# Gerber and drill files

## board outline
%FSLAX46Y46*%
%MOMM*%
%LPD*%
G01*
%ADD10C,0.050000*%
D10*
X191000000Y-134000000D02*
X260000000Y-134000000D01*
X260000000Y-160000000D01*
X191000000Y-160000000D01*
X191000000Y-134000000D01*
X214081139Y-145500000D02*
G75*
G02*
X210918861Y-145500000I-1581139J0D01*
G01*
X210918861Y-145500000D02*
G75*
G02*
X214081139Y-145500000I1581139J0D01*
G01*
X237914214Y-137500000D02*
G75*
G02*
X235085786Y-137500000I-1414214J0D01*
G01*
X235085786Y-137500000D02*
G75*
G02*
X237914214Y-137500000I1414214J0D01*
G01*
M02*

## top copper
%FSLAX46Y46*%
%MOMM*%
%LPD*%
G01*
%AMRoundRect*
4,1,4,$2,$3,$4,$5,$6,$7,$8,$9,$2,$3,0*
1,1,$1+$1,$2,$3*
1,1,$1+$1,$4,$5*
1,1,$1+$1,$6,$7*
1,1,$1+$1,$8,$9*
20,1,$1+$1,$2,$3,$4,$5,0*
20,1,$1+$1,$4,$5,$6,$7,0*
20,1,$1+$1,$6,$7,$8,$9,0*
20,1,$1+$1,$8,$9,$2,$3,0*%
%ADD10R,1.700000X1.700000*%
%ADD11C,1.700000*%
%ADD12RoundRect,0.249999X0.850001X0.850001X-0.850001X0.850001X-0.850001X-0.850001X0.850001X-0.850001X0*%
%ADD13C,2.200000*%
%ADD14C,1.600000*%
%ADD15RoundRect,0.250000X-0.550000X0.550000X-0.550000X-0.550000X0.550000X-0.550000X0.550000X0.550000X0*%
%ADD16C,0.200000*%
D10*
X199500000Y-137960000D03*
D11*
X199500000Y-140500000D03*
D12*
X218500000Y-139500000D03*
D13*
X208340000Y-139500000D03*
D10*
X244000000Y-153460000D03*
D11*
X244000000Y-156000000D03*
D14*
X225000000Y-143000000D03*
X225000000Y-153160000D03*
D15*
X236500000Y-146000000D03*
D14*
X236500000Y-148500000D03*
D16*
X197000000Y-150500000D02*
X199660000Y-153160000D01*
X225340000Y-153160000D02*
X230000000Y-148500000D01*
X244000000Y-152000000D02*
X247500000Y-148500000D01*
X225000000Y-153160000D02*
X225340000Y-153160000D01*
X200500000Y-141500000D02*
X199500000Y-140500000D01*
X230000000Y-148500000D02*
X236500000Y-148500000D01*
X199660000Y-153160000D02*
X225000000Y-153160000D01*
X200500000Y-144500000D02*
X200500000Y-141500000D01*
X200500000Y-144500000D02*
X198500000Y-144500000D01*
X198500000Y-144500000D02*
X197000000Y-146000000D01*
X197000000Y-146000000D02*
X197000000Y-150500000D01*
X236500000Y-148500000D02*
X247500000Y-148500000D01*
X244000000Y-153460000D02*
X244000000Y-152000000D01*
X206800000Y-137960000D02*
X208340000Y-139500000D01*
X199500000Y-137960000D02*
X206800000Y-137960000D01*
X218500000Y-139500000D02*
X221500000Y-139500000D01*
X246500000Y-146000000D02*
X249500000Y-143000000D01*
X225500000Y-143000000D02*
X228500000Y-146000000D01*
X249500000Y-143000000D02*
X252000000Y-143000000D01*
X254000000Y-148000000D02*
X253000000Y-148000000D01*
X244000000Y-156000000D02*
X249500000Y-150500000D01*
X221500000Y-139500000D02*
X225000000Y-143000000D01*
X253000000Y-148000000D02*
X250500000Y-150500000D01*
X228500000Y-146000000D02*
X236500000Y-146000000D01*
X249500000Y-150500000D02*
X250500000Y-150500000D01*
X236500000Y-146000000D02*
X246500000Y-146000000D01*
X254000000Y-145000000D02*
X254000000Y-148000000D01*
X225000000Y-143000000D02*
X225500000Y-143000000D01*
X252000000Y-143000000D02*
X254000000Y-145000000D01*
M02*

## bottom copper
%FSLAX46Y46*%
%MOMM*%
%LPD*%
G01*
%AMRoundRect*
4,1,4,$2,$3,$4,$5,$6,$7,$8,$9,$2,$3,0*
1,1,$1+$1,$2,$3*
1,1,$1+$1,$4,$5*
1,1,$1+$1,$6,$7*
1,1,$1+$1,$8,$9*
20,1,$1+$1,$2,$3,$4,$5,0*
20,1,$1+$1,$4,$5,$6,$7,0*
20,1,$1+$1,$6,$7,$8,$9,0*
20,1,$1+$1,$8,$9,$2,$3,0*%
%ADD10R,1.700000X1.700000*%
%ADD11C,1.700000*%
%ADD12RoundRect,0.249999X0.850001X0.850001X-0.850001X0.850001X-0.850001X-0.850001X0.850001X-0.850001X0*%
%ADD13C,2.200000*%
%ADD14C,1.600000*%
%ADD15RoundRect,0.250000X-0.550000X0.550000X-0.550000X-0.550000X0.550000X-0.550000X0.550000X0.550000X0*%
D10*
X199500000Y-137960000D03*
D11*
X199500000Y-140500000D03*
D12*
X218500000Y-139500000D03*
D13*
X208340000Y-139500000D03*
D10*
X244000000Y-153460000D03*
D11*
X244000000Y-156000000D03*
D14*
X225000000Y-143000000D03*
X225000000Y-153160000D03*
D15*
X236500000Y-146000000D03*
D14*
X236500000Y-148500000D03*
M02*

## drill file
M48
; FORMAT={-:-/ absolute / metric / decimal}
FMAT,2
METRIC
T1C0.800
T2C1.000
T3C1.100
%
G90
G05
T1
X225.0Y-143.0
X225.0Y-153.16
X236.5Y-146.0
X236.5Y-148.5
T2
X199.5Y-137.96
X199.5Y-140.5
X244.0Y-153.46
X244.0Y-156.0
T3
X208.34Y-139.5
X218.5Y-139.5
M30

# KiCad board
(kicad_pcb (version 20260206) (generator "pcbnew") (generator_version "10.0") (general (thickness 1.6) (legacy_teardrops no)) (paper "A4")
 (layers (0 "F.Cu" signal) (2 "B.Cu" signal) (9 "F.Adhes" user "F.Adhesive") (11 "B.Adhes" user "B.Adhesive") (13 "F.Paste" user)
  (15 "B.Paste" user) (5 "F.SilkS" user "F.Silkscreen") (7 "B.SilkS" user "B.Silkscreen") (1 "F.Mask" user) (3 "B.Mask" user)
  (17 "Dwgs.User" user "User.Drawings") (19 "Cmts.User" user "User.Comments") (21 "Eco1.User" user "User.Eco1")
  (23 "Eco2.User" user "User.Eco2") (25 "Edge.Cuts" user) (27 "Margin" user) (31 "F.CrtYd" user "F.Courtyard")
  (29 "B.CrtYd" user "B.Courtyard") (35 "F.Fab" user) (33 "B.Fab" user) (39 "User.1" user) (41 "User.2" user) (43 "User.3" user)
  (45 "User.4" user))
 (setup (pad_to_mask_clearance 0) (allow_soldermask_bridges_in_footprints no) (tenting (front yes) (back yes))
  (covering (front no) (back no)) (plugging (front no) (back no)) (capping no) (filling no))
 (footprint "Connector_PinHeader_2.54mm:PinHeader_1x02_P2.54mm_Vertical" (layer "F.Cu") (at 199.5 137.96)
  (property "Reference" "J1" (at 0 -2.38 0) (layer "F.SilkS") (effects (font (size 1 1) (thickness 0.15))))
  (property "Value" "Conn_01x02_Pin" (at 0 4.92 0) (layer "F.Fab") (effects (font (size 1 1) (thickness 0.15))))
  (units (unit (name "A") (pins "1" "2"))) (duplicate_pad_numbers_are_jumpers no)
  (pad "1" thru_hole rect (at 0 0) (size 1.7 1.7) (drill 1) (layers "*.Cu" "*.Mask") (remove_unused_layers no) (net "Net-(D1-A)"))
  (pad "2" thru_hole circle (at 0 2.54) (size 1.7 1.7) (drill 1) (layers "*.Cu" "*.Mask") (remove_unused_layers no) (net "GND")))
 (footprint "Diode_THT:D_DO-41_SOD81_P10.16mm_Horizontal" (layer "F.Cu") (at 218.5 139.5 180)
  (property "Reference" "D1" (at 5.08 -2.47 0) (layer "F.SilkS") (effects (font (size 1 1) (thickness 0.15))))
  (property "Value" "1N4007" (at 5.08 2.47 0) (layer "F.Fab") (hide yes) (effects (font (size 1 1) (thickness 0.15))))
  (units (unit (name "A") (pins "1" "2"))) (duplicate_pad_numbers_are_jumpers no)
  (pad "1" thru_hole roundrect (at 0 0 180) (size 2.2 2.2) (drill 1.1) (layers "*.Cu" "*.Mask") (remove_unused_layers no)
   (roundrect_rratio 0.113636) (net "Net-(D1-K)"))
  (pad "2" thru_hole circle (at 10.16 0 180) (size 2.2 2.2) (drill 1.1) (layers "*.Cu" "*.Mask") (remove_unused_layers no)
   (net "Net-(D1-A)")))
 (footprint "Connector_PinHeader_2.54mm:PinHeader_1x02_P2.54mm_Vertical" (layer "F.Cu") (at 244 153.46)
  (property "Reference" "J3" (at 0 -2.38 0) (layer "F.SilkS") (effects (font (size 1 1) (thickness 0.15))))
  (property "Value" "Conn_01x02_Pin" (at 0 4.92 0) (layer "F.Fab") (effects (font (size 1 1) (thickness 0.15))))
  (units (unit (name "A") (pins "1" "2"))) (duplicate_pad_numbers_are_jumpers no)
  (pad "1" thru_hole rect (at 0 0) (size 1.7 1.7) (drill 1) (layers "*.Cu" "*.Mask") (remove_unused_layers no) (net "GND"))
  (pad "2" thru_hole circle (at 0 2.54) (size 1.7 1.7) (drill 1) (layers "*.Cu" "*.Mask") (remove_unused_layers no) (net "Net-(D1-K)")))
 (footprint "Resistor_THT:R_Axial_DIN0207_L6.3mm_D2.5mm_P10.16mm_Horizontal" (layer "F.Cu") (at 225 143 -90)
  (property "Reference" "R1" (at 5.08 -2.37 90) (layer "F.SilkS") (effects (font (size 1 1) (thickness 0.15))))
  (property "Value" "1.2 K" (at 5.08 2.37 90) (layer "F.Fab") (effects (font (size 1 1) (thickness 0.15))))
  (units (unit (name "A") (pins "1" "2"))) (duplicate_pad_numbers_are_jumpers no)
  (pad "1" thru_hole circle (at 0 0 270) (size 1.6 1.6) (drill 0.8) (layers "*.Cu" "*.Mask") (remove_unused_layers no) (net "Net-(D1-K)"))
  (pad "2" thru_hole circle (at 10.16 0 270) (size 1.6 1.6) (drill 0.8) (layers "*.Cu" "*.Mask") (remove_unused_layers no) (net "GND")))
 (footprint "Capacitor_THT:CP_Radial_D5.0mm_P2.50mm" (layer "F.Cu") (at 236.5 146 -90)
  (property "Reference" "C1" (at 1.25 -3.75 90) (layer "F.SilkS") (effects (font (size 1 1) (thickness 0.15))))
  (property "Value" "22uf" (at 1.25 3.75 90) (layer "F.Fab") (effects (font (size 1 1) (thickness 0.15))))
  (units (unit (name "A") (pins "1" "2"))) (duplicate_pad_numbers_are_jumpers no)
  (pad "1" thru_hole roundrect (at 0 0 270) (size 1.6 1.6) (drill 0.8) (layers "*.Cu" "*.Mask") (remove_unused_layers no)
   (roundrect_rratio 0.15625) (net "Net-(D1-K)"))
  (pad "2" thru_hole circle (at 2.5 0 270) (size 1.6 1.6) (drill 0.8) (layers "*.Cu" "*.Mask") (remove_unused_layers no) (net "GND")))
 (gr_rect (start 191 134) (end 260 160) (stroke (width 0.05) (type default)) (fill no) (layer "Edge.Cuts"))
 (gr_circle (center 212.5 145.5) (end 214 146) (stroke (width 0.05) (type default)) (fill no) (layer "Edge.Cuts"))
 (gr_circle (center 236.5 137.5) (end 237.5 138.5) (stroke (width 0.05) (type default)) (fill no) (layer "Edge.Cuts"))
 (segment (start 197 150.5) (end 199.66 153.16) (width 0.2) (layer "F.Cu") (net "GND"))
 (segment (start 225.34 153.16) (end 230 148.5) (width 0.2) (layer "F.Cu") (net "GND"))
 (segment (start 244 152) (end 247.5 148.5) (width 0.2) (layer "F.Cu") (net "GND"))
 (segment (start 225 153.16) (end 225.34 153.16) (width 0.2) (layer "F.Cu") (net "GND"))
 (segment (start 200.5 141.5) (end 199.5 140.5) (width 0.2) (layer "F.Cu") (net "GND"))
 (segment (start 230 148.5) (end 236.5 148.5) (width 0.2) (layer "F.Cu") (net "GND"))
 (segment (start 199.66 153.16) (end 225 153.16) (width 0.2) (layer "F.Cu") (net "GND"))
 (segment (start 200.5 144.5) (end 200.5 141.5) (width 0.2) (layer "F.Cu") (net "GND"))
 (segment (start 200.5 144.5) (end 198.5 144.5) (width 0.2) (layer "F.Cu") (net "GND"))
 (segment (start 198.5 144.5) (end 197 146) (width 0.2) (layer "F.Cu") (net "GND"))
 (segment (start 197 146) (end 197 150.5) (width 0.2) (layer "F.Cu") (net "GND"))
 (segment (start 236.5 148.5) (end 247.5 148.5) (width 0.2) (layer "F.Cu") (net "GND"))
 (segment (start 244 153.46) (end 244 152) (width 0.2) (layer "F.Cu") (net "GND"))
 (segment (start 206.8 137.96) (end 208.34 139.5) (width 0.2) (layer "F.Cu") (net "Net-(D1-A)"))
 (segment (start 199.5 137.96) (end 206.8 137.96) (width 0.2) (layer "F.Cu") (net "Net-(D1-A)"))
 (segment (start 218.5 139.5) (end 221.5 139.5) (width 0.2) (layer "F.Cu") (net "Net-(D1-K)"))
 (segment (start 246.5 146) (end 249.5 143) (width 0.2) (layer "F.Cu") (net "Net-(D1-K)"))
 (segment (start 225.5 143) (end 228.5 146) (width 0.2) (layer "F.Cu") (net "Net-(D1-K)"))
 (segment (start 249.5 143) (end 252 143) (width 0.2) (layer "F.Cu") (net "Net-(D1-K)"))
 (segment (start 254 148) (end 253 148) (width 0.2) (layer "F.Cu") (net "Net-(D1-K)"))
 (segment (start 244 156) (end 249.5 150.5) (width 0.2) (layer "F.Cu") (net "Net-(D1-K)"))
 (segment (start 221.5 139.5) (end 225 143) (width 0.2) (layer "F.Cu") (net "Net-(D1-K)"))
 (segment (start 253 148) (end 250.5 150.5) (width 0.2) (layer "F.Cu") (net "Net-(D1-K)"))
 (segment (start 228.5 146) (end 236.5 146) (width 0.2) (layer "F.Cu") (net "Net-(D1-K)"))
 (segment (start 249.5 150.5) (end 250.5 150.5) (width 0.2) (layer "F.Cu") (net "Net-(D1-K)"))
 (segment (start 236.5 146) (end 246.5 146) (width 0.2) (layer "F.Cu") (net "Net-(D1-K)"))
 (segment (start 254 145) (end 254 148) (width 0.2) (layer "F.Cu") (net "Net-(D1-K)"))
 (segment (start 225 143) (end 225.5 143) (width 0.2) (layer "F.Cu") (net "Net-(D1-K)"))
 (segment (start 252 143) (end 254 145) (width 0.2) (layer "F.Cu") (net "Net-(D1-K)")))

